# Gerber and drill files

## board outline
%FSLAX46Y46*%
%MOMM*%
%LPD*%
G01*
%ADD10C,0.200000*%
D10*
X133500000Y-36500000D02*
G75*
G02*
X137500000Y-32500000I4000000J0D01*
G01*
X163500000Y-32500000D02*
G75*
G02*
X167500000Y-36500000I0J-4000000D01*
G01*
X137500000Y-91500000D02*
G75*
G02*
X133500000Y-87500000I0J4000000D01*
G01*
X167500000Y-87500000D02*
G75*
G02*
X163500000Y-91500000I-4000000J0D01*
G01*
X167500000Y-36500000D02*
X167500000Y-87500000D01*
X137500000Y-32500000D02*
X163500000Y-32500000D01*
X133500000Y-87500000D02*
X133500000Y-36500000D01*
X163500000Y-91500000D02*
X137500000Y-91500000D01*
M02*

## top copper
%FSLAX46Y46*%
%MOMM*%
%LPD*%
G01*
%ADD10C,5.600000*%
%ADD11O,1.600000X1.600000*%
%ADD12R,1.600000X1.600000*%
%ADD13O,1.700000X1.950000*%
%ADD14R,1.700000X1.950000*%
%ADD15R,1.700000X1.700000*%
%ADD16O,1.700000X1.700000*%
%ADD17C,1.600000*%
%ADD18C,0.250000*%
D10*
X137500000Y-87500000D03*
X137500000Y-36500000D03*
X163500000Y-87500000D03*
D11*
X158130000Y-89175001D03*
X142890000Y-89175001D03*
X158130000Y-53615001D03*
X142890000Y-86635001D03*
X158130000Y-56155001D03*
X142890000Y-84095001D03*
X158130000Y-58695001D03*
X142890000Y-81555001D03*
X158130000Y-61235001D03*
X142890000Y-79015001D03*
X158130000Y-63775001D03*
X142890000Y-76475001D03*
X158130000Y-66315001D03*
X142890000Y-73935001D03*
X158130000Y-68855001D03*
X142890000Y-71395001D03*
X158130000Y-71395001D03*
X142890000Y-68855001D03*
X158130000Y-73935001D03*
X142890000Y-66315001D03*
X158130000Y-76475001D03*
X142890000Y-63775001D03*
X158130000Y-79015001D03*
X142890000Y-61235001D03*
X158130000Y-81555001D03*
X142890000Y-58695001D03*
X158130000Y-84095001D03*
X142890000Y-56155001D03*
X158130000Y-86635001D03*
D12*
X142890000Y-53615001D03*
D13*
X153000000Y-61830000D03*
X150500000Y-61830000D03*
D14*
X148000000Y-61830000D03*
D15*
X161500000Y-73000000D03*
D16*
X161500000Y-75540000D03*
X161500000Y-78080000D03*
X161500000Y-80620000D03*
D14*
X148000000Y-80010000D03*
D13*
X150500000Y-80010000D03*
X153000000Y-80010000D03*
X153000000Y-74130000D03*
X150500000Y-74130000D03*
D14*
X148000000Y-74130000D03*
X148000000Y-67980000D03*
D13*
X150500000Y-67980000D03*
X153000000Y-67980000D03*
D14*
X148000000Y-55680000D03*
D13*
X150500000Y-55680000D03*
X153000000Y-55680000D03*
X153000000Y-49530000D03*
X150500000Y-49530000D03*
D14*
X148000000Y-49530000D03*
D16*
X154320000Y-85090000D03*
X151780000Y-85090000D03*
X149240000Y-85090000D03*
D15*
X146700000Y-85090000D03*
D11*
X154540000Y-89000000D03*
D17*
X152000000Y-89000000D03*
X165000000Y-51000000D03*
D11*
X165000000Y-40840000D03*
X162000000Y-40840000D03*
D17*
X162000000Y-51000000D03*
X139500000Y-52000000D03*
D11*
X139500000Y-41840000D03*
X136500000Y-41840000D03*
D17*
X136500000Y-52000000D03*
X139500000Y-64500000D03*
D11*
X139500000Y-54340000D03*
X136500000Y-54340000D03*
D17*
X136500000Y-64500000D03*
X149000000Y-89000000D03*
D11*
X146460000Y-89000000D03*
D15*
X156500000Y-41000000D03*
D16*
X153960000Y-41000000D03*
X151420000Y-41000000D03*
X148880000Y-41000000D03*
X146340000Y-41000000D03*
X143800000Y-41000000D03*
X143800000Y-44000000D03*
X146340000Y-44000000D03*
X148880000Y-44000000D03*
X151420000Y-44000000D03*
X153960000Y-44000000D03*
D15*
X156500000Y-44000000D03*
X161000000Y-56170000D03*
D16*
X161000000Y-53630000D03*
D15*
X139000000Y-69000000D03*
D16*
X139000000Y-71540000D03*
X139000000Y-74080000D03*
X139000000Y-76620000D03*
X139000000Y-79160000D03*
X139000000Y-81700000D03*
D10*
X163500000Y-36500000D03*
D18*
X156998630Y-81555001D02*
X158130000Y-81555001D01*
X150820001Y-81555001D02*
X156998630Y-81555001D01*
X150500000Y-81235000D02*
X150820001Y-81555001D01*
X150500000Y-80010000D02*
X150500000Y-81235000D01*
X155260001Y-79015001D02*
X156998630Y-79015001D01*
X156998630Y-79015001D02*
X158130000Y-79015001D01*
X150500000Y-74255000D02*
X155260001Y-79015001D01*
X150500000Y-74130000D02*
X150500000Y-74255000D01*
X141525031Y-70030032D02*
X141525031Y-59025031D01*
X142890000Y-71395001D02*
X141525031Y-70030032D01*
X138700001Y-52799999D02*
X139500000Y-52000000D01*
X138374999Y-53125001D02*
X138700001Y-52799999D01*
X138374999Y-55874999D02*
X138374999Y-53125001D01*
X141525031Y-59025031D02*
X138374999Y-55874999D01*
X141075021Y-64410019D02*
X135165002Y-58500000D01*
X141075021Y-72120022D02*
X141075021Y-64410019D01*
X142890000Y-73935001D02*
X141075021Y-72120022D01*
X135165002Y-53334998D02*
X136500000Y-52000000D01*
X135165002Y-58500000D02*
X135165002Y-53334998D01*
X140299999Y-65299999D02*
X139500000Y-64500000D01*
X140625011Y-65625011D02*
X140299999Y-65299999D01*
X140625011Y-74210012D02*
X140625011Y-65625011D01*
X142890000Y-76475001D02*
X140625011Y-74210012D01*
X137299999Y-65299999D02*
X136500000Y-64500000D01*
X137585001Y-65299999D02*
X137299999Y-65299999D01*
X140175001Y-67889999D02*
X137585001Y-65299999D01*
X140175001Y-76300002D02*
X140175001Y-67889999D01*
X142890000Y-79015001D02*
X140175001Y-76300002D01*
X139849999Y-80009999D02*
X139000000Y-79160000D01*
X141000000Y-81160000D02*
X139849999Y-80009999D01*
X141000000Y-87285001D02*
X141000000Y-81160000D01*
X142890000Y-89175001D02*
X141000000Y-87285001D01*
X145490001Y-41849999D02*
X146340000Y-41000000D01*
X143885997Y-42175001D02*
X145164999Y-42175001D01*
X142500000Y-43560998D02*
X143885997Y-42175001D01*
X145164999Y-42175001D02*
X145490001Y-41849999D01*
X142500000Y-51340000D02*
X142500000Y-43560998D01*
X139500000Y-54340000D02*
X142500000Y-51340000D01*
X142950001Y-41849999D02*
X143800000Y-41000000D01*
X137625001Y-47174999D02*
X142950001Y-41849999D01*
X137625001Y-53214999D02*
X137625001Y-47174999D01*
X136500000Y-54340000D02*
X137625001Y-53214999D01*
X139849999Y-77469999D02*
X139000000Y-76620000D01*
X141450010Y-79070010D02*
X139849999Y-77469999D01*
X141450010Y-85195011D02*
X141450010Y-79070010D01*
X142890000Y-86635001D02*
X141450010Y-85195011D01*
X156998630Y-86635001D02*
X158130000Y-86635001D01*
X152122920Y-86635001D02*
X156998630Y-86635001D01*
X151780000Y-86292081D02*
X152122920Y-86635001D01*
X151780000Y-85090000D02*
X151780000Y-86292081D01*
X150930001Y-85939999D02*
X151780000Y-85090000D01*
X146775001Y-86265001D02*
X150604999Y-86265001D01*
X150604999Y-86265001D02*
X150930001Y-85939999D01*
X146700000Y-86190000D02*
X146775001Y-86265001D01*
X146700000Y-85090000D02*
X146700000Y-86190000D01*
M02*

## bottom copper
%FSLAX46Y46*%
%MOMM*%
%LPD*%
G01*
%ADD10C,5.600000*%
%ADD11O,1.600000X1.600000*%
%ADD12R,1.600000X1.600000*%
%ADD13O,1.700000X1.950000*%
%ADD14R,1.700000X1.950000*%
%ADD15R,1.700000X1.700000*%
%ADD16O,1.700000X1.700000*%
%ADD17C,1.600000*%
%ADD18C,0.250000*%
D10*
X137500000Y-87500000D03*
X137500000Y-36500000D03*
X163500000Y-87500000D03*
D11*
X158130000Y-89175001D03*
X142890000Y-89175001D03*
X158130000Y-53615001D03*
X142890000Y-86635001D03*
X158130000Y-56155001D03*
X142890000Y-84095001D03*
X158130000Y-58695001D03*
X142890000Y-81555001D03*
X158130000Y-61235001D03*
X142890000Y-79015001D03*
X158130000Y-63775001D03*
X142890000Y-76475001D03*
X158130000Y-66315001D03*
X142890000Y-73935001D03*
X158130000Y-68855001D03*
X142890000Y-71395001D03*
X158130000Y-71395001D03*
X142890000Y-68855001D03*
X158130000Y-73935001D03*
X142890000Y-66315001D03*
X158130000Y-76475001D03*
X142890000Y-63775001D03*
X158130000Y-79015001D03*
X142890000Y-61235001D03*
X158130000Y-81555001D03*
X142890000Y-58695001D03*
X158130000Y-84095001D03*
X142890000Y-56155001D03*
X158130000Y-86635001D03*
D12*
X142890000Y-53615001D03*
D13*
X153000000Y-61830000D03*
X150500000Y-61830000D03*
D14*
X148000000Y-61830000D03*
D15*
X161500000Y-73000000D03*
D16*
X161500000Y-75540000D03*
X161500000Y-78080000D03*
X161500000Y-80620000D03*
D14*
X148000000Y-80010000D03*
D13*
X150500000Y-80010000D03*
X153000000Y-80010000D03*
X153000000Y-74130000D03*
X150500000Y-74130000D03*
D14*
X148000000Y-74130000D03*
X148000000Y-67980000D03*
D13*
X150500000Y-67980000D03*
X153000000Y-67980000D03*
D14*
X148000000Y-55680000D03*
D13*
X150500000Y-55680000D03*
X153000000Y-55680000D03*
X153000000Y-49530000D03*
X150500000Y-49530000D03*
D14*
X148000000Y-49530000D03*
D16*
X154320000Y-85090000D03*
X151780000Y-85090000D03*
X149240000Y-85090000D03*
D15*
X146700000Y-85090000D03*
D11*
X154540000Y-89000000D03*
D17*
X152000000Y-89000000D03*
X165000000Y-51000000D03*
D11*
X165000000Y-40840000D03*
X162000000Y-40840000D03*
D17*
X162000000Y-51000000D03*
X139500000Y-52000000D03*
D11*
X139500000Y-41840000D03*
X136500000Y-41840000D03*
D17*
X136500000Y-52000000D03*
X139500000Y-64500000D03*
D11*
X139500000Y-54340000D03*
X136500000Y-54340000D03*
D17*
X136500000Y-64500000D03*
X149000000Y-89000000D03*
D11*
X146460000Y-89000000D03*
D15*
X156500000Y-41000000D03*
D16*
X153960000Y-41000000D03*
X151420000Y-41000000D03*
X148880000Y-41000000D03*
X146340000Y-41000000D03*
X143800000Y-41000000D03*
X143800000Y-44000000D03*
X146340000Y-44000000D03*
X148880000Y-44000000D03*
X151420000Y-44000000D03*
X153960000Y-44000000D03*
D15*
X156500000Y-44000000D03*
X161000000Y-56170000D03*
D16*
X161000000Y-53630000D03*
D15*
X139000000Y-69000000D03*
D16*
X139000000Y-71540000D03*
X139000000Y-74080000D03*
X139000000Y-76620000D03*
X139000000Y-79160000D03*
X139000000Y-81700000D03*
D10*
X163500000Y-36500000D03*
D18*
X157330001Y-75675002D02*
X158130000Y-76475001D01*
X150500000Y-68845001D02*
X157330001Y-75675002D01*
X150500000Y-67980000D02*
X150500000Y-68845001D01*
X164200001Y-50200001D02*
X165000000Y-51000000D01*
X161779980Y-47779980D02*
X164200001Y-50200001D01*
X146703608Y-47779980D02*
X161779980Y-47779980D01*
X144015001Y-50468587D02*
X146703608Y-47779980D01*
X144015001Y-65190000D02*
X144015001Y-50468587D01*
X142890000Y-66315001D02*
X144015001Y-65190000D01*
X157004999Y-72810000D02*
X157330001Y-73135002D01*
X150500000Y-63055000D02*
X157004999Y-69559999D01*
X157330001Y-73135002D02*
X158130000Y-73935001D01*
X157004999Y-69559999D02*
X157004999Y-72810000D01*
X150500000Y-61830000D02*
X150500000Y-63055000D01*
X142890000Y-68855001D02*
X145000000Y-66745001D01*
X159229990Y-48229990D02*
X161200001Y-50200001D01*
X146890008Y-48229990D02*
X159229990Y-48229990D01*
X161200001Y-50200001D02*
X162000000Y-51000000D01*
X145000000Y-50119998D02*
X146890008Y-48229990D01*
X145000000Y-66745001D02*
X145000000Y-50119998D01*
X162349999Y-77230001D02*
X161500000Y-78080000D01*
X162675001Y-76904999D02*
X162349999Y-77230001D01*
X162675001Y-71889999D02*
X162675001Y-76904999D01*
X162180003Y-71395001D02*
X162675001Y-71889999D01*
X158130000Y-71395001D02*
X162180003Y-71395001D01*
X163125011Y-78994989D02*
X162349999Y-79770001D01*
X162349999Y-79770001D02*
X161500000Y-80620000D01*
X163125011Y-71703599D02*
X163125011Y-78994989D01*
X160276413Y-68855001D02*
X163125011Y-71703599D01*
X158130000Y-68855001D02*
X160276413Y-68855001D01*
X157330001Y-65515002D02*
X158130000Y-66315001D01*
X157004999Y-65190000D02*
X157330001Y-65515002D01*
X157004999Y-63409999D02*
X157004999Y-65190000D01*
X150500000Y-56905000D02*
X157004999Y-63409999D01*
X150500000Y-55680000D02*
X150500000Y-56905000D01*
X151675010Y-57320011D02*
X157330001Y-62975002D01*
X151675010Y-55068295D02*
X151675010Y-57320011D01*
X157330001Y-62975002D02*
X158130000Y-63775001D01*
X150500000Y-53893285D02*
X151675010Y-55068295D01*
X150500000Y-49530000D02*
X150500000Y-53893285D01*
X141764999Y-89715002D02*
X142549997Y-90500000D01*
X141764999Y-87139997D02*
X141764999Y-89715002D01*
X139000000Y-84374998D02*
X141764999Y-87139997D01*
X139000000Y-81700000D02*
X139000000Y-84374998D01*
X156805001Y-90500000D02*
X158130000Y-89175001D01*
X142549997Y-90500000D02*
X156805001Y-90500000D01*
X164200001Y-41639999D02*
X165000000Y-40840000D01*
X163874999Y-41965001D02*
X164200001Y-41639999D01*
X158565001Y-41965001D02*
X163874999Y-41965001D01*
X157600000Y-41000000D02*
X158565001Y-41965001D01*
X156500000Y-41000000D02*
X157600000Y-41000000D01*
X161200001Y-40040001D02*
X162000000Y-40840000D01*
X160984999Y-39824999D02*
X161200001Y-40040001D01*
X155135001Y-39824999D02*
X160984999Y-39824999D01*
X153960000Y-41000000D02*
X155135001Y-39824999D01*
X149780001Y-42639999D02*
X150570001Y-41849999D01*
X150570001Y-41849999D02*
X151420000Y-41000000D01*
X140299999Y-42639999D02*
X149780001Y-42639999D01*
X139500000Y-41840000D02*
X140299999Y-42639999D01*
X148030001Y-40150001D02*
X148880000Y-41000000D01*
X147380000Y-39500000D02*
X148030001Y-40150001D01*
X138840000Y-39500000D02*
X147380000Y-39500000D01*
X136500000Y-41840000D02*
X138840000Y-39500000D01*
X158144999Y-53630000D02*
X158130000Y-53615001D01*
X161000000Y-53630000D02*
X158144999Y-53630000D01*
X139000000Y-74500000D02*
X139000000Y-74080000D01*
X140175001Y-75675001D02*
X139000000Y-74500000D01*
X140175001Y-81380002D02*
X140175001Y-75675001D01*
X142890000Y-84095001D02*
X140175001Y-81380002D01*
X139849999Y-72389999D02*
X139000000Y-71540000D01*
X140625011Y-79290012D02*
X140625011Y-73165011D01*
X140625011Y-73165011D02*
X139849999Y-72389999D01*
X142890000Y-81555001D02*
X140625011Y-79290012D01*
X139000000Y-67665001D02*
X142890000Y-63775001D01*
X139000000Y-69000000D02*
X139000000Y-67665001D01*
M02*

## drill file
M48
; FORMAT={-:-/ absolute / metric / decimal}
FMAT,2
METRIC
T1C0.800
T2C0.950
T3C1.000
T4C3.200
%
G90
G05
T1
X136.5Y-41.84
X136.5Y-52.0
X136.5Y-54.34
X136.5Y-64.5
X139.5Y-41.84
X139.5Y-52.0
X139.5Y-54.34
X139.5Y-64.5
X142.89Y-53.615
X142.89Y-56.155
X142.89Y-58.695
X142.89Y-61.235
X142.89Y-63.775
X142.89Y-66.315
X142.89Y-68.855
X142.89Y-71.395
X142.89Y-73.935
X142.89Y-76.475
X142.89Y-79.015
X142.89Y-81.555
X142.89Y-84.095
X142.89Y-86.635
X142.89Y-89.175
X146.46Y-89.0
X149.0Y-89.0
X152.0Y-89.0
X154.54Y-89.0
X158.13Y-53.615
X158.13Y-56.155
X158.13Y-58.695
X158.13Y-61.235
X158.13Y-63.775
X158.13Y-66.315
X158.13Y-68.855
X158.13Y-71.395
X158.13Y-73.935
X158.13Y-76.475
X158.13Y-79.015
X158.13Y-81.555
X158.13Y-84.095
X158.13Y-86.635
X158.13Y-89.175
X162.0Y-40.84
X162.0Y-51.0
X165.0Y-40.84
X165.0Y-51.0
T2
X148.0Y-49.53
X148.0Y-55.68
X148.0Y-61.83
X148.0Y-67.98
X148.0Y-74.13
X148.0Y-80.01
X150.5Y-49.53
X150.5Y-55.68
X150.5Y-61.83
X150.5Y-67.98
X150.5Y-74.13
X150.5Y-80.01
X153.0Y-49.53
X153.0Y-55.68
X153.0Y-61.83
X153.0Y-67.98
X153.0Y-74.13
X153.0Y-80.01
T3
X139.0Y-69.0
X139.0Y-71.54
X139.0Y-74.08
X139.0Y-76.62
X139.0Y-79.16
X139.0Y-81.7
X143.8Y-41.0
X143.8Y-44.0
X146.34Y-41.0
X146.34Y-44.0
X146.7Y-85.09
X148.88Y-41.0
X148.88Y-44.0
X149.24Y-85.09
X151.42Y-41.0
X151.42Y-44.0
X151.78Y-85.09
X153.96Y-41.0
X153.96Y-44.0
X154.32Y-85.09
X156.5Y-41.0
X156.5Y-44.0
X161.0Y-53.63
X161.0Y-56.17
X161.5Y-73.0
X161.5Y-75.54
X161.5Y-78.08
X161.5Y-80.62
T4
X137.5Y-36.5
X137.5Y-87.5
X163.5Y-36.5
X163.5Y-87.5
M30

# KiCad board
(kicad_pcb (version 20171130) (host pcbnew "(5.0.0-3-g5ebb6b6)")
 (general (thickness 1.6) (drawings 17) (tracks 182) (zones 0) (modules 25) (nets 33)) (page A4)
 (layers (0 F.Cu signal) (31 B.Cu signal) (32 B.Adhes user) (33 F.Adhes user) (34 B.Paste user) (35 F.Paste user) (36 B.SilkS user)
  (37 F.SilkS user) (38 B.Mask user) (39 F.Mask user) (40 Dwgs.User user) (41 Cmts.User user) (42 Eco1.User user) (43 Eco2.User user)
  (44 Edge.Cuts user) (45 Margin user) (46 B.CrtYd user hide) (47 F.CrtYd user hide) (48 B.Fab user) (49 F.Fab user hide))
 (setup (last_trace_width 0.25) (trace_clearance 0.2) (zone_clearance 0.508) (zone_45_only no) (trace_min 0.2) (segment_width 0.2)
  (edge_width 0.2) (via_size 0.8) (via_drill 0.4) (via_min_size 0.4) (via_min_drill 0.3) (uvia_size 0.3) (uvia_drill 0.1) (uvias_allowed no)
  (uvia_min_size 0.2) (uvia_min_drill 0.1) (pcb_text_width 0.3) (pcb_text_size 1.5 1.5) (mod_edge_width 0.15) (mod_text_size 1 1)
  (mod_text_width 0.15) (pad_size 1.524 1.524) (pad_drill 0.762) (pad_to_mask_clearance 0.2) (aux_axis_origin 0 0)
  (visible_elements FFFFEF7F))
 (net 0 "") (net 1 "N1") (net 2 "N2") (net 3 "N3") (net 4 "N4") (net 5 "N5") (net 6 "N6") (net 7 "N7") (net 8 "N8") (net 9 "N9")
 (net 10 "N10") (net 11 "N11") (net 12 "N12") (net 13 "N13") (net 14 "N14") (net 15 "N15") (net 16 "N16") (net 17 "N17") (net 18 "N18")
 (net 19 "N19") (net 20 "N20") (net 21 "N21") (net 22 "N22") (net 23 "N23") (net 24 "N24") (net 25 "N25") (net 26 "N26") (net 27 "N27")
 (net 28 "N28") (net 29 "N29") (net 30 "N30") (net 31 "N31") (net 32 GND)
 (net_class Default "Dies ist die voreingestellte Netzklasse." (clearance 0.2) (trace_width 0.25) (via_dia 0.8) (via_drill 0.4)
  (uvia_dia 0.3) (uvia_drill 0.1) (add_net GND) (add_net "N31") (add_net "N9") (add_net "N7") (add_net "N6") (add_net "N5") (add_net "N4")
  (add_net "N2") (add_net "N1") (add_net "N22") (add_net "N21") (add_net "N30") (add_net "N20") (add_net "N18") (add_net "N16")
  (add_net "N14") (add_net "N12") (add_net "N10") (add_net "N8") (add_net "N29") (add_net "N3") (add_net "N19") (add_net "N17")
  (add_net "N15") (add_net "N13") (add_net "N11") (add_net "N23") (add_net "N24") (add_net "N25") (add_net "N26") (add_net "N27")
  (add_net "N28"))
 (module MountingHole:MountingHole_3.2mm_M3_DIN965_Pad (layer F.Cu) (at 137.5 87.5)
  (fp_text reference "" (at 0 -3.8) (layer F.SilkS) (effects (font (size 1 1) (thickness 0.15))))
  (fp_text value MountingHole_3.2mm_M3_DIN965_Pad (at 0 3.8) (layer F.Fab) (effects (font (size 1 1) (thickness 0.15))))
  (pad 1 thru_hole circle (at 0 0) (size 5.6 5.6) (drill 3.2) (layers *.Cu *.Mask)))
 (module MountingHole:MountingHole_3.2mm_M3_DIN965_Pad (layer F.Cu) (at 137.5 36.5)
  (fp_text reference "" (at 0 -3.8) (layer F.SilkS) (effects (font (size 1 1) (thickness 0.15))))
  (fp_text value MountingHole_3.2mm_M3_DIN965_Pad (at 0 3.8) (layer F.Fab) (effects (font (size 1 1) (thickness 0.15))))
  (pad 1 thru_hole circle (at 0 0) (size 5.6 5.6) (drill 3.2) (layers *.Cu *.Mask)))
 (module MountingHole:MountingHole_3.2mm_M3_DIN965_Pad (layer F.Cu) (at 163.5 87.5)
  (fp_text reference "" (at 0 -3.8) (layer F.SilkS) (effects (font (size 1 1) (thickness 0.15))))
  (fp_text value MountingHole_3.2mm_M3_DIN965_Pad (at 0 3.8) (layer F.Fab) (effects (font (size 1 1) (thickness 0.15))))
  (pad 1 thru_hole circle (at 0 0) (size 5.6 5.6) (drill 3.2) (layers *.Cu *.Mask)))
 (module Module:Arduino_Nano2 (layer F.Cu) (at 142.89 53.615001)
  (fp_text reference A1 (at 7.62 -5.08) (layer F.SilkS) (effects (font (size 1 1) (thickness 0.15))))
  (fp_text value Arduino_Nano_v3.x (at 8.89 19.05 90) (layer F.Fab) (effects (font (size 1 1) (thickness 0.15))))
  (pad 16 thru_hole oval (at 15.24 35.56) (size 1.6 1.6) (drill 0.8) (layers *.Cu *.Mask) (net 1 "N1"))
  (pad 15 thru_hole oval (at 0 35.56) (size 1.6 1.6) (drill 0.8) (layers *.Cu *.Mask) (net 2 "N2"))
  (pad 30 thru_hole oval (at 15.24 0) (size 1.6 1.6) (drill 0.8) (layers *.Cu *.Mask) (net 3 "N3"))
  (pad 14 thru_hole oval (at 0 33.02) (size 1.6 1.6) (drill 0.8) (layers *.Cu *.Mask) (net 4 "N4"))
  (pad 29 thru_hole oval (at 15.24 2.54) (size 1.6 1.6) (drill 0.8) (layers *.Cu *.Mask))
  (pad 13 thru_hole oval (at 0 30.48) (size 1.6 1.6) (drill 0.8) (layers *.Cu *.Mask) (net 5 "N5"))
  (pad 28 thru_hole oval (at 15.24 5.08) (size 1.6 1.6) (drill 0.8) (layers *.Cu *.Mask))
  (pad 12 thru_hole oval (at 0 27.94) (size 1.6 1.6) (drill 0.8) (layers *.Cu *.Mask) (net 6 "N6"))
  (pad 27 thru_hole oval (at 15.24 7.62) (size 1.6 1.6) (drill 0.8) (layers *.Cu *.Mask))
  (pad 11 thru_hole oval (at 0 25.4) (size 1.6 1.6) (drill 0.8) (layers *.Cu *.Mask) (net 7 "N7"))
  (pad 26 thru_hole oval (at 15.24 10.16) (size 1.6 1.6) (drill 0.8) (layers *.Cu *.Mask) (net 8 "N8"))
  (pad 10 thru_hole oval (at 0 22.86) (size 1.6 1.6) (drill 0.8) (layers *.Cu *.Mask) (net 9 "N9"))
  (pad 25 thru_hole oval (at 15.24 12.7) (size 1.6 1.6) (drill 0.8) (layers *.Cu *.Mask) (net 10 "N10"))
  (pad 9 thru_hole oval (at 0 20.32) (size 1.6 1.6) (drill 0.8) (layers *.Cu *.Mask) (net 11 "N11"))
  (pad 24 thru_hole oval (at 15.24 15.24) (size 1.6 1.6) (drill 0.8) (layers *.Cu *.Mask) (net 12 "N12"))
  (pad 8 thru_hole oval (at 0 17.78) (size 1.6 1.6) (drill 0.8) (layers *.Cu *.Mask) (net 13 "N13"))
  (pad 23 thru_hole oval (at 15.24 17.78) (size 1.6 1.6) (drill 0.8) (layers *.Cu *.Mask) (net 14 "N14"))
  (pad 7 thru_hole oval (at 0 15.24) (size 1.6 1.6) (drill 0.8) (layers *.Cu *.Mask) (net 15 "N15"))
  (pad 22 thru_hole oval (at 15.24 20.32) (size 1.6 1.6) (drill 0.8) (layers *.Cu *.Mask) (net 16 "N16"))
  (pad 6 thru_hole oval (at 0 12.7) (size 1.6 1.6) (drill 0.8) (layers *.Cu *.Mask) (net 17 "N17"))
  (pad 21 thru_hole oval (at 15.24 22.86) (size 1.6 1.6) (drill 0.8) (layers *.Cu *.Mask) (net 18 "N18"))
  (pad 5 thru_hole oval (at 0 10.16) (size 1.6 1.6) (drill 0.8) (layers *.Cu *.Mask) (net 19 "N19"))
  (pad 20 thru_hole oval (at 15.24 25.4) (size 1.6 1.6) (drill 0.8) (layers *.Cu *.Mask) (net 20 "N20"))
  (pad 4 thru_hole oval (at 0 7.62) (size 1.6 1.6) (drill 0.8) (layers *.Cu *.Mask))
  (pad 19 thru_hole oval (at 15.24 27.94) (size 1.6 1.6) (drill 0.8) (layers *.Cu *.Mask) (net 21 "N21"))
  (pad 3 thru_hole oval (at 0 5.08) (size 1.6 1.6) (drill 0.8) (layers *.Cu *.Mask))
  (pad 18 thru_hole oval (at 15.24 30.48) (size 1.6 1.6) (drill 0.8) (layers *.Cu *.Mask))
  (pad 2 thru_hole oval (at 0 2.54) (size 1.6 1.6) (drill 0.8) (layers *.Cu *.Mask))
  (pad 17 thru_hole oval (at 15.24 33.02) (size 1.6 1.6) (drill 0.8) (layers *.Cu *.Mask) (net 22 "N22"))
  (pad 1 thru_hole rect (at 0 0) (size 1.6 1.6) (drill 0.8) (layers *.Cu *.Mask)))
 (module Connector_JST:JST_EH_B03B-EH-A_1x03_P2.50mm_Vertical (layer F.Cu) (at 148 61.83)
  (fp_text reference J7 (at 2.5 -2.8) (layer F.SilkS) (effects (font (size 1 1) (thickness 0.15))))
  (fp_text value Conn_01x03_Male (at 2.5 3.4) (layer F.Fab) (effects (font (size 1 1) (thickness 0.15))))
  (pad 3 thru_hole oval (at 5 0) (size 1.7 1.95) (drill 0.95) (layers *.Cu *.Mask))
  (pad 2 thru_hole oval (at 2.5 0) (size 1.7 1.95) (drill 0.95) (layers *.Cu *.Mask) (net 16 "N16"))
  (pad 1 thru_hole rect (at 0 0) (size 1.7 1.95) (drill 0.95) (layers *.Cu *.Mask)))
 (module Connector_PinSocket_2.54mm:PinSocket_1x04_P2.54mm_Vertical (layer F.Cu) (at 161.5 73)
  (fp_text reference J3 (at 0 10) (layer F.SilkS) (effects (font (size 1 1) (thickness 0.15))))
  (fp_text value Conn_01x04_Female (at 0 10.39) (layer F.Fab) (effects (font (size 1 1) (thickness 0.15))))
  (pad 1 thru_hole rect (at 0 0) (size 1.7 1.7) (drill 1) (layers *.Cu *.Mask))
  (pad 2 thru_hole oval (at 0 2.54) (size 1.7 1.7) (drill 1) (layers *.Cu *.Mask))
  (pad 3 thru_hole oval (at 0 5.08) (size 1.7 1.7) (drill 1) (layers *.Cu *.Mask) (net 14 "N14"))
  (pad 4 thru_hole oval (at 0 7.62) (size 1.7 1.7) (drill 1) (layers *.Cu *.Mask) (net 12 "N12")))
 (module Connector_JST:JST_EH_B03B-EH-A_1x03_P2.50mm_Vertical (layer F.Cu) (at 148 80.01)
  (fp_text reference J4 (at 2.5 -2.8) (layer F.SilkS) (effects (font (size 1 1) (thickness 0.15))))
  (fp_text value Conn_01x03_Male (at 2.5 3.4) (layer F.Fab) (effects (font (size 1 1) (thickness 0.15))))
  (pad 1 thru_hole rect (at 0 0) (size 1.7 1.95) (drill 0.95) (layers *.Cu *.Mask))
  (pad 2 thru_hole oval (at 2.5 0) (size 1.7 1.95) (drill 0.95) (layers *.Cu *.Mask) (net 21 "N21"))
  (pad 3 thru_hole oval (at 5 0) (size 1.7 1.95) (drill 0.95) (layers *.Cu *.Mask)))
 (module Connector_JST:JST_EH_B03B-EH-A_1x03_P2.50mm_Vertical (layer F.Cu) (at 148 74.13)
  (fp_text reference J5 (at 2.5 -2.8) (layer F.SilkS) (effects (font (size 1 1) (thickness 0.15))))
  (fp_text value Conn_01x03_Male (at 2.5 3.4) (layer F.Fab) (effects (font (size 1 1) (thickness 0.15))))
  (pad 3 thru_hole oval (at 5 0) (size 1.7 1.95) (drill 0.95) (layers *.Cu *.Mask))
  (pad 2 thru_hole oval (at 2.5 0) (size 1.7 1.95) (drill 0.95) (layers *.Cu *.Mask) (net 20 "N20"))
  (pad 1 thru_hole rect (at 0 0) (size 1.7 1.95) (drill 0.95) (layers *.Cu *.Mask)))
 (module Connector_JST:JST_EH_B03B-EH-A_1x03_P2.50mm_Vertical (layer F.Cu) (at 148 67.98)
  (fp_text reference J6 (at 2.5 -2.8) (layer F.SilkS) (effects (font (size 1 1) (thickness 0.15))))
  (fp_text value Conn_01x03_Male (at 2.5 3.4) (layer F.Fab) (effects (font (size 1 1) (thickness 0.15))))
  (pad 1 thru_hole rect (at 0 0) (size 1.7 1.95) (drill 0.95) (layers *.Cu *.Mask))
  (pad 2 thru_hole oval (at 2.5 0) (size 1.7 1.95) (drill 0.95) (layers *.Cu *.Mask) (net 18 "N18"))
  (pad 3 thru_hole oval (at 5 0) (size 1.7 1.95) (drill 0.95) (layers *.Cu *.Mask)))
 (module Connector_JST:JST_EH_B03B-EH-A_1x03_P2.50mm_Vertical (layer F.Cu) (at 148 55.68)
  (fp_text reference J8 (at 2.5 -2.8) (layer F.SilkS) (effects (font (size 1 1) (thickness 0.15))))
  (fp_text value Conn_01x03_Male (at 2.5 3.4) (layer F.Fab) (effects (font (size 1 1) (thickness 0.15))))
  (pad 1 thru_hole rect (at 0 0) (size 1.7 1.95) (drill 0.95) (layers *.Cu *.Mask))
  (pad 2 thru_hole oval (at 2.5 0) (size 1.7 1.95) (drill 0.95) (layers *.Cu *.Mask) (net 10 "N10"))
  (pad 3 thru_hole oval (at 5 0) (size 1.7 1.95) (drill 0.95) (layers *.Cu *.Mask)))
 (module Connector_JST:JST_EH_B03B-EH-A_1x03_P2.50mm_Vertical (layer F.Cu) (at 148 49.53)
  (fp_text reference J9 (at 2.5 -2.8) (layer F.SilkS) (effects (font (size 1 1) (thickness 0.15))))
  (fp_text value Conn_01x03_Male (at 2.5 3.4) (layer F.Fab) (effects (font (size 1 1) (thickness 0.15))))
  (pad 3 thru_hole oval (at 5 0) (size 1.7 1.95) (drill 0.95) (layers *.Cu *.Mask))
  (pad 2 thru_hole oval (at 2.5 0) (size 1.7 1.95) (drill 0.95) (layers *.Cu *.Mask) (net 8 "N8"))
  (pad 1 thru_hole rect (at 0 0) (size 1.7 1.95) (drill 0.95) (layers *.Cu *.Mask)))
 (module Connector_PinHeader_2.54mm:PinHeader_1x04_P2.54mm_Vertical (layer F.Cu) (at 146.7 85.09 90)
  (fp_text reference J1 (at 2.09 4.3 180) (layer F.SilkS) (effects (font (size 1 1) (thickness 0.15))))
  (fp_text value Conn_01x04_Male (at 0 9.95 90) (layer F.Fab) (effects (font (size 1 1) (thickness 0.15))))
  (pad 4 thru_hole oval (at 0 7.62 90) (size 1.7 1.7) (drill 1) (layers *.Cu *.Mask))
  (pad 3 thru_hole oval (at 0 5.08 90) (size 1.7 1.7) (drill 1) (layers *.Cu *.Mask) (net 22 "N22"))
  (pad 2 thru_hole oval (at 0 2.54 90) (size 1.7 1.7) (drill 1) (layers *.Cu *.Mask))
  (pad 1 thru_hole rect (at 0 0 90) (size 1.7 1.7) (drill 1) (layers *.Cu *.Mask) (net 22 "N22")))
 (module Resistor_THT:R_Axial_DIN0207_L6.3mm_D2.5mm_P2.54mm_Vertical (layer F.Cu) (at 152 89)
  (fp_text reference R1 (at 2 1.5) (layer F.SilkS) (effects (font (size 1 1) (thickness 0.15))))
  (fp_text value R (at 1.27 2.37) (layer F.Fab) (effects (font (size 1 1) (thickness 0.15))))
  (pad 2 thru_hole oval (at 2.54 0) (size 1.6 1.6) (drill 0.8) (layers *.Cu *.Mask))
  (pad 1 thru_hole circle (at 0 0) (size 1.6 1.6) (drill 0.8) (layers *.Cu *.Mask)))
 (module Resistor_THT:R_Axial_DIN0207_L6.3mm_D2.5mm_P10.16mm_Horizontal (layer F.Cu) (at 165 51 90)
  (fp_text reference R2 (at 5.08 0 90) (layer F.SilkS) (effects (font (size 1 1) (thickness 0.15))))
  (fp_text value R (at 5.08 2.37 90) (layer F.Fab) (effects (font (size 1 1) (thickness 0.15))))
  (pad 1 thru_hole circle (at 0 0 90) (size 1.6 1.6) (drill 0.8) (layers *.Cu *.Mask) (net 17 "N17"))
  (pad 2 thru_hole oval (at 10.16 0 90) (size 1.6 1.6) (drill 0.8) (layers *.Cu *.Mask) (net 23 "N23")))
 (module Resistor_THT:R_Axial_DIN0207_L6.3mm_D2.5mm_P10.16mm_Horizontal (layer F.Cu) (at 162 51 90)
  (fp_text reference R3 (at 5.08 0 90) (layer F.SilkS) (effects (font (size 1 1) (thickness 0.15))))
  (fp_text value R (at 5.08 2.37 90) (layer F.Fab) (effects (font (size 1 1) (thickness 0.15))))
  (pad 2 thru_hole oval (at 10.16 0 90) (size 1.6 1.6) (drill 0.8) (layers *.Cu *.Mask) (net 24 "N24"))
  (pad 1 thru_hole circle (at 0 0 90) (size 1.6 1.6) (drill 0.8) (layers *.Cu *.Mask) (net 15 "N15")))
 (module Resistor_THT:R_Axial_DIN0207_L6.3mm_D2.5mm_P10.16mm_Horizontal (layer F.Cu) (at 139.5 52 90)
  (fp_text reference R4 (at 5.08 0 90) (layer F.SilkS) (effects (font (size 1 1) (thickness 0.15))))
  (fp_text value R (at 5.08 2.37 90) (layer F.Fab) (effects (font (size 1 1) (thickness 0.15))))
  (pad 1 thru_hole circle (at 0 0 90) (size 1.6 1.6) (drill 0.8) (layers *.Cu *.Mask) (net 13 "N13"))
  (pad 2 thru_hole oval (at 10.16 0 90) (size 1.6 1.6) (drill 0.8) (layers *.Cu *.Mask) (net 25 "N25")))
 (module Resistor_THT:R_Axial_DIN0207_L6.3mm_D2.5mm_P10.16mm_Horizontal (layer F.Cu) (at 136.5 52 90)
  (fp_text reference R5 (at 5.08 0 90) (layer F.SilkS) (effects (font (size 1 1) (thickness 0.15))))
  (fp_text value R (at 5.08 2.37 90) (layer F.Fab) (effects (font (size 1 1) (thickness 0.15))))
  (pad 2 thru_hole oval (at 10.16 0 90) (size 1.6 1.6) (drill 0.8) (layers *.Cu *.Mask) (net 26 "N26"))
  (pad 1 thru_hole circle (at 0 0 90) (size 1.6 1.6) (drill 0.8) (layers *.Cu *.Mask) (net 11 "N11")))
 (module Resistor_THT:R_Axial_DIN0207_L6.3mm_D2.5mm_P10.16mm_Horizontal (layer F.Cu) (at 139.5 64.5 90)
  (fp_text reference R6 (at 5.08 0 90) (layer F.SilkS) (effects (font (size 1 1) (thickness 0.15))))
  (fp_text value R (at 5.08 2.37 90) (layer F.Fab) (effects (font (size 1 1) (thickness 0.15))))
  (pad 1 thru_hole circle (at 0 0 90) (size 1.6 1.6) (drill 0.8) (layers *.Cu *.Mask) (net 9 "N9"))
  (pad 2 thru_hole oval (at 10.16 0 90) (size 1.6 1.6) (drill 0.8) (layers *.Cu *.Mask) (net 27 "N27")))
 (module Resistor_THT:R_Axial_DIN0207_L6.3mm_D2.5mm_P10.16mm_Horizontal (layer F.Cu) (at 136.5 64.5 90)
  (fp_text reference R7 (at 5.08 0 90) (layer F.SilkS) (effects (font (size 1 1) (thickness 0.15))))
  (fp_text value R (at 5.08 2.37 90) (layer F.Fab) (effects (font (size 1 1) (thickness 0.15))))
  (pad 2 thru_hole oval (at 10.16 0 90) (size 1.6 1.6) (drill 0.8) (layers *.Cu *.Mask) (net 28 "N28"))
  (pad 1 thru_hole circle (at 0 0 90) (size 1.6 1.6) (drill 0.8) (layers *.Cu *.Mask) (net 7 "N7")))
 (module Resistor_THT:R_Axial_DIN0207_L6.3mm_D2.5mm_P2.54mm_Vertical (layer F.Cu) (at 149 89 180)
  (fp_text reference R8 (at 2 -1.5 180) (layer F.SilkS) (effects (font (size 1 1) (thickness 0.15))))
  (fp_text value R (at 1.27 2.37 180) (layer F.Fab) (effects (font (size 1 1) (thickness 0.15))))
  (pad 1 thru_hole circle (at 0 0 180) (size 1.6 1.6) (drill 0.8) (layers *.Cu *.Mask))
  (pad 2 thru_hole oval (at 2.54 0 180) (size 1.6 1.6) (drill 0.8) (layers *.Cu *.Mask)))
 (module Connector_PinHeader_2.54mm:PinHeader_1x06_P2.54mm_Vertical (layer F.Cu) (at 156.5 41 270)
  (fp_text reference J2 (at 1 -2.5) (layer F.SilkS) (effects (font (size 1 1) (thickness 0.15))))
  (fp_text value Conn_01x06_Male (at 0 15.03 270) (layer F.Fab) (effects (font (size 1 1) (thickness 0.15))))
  (pad 1 thru_hole rect (at 0 0 270) (size 1.7 1.7) (drill 1) (layers *.Cu *.Mask) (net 23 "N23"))
  (pad 2 thru_hole oval (at 0 2.54 270) (size 1.7 1.7) (drill 1) (layers *.Cu *.Mask) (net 24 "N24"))
  (pad 3 thru_hole oval (at 0 5.08 270) (size 1.7 1.7) (drill 1) (layers *.Cu *.Mask) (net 25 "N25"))
  (pad 4 thru_hole oval (at 0 7.62 270) (size 1.7 1.7) (drill 1) (layers *.Cu *.Mask) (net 26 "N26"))
  (pad 5 thru_hole oval (at 0 10.16 270) (size 1.7 1.7) (drill 1) (layers *.Cu *.Mask) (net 27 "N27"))
  (pad 6 thru_hole oval (at 0 12.7 270) (size 1.7 1.7) (drill 1) (layers *.Cu *.Mask) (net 28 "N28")))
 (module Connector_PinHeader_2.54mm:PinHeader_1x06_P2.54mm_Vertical (layer F.Cu) (at 156.5 44 270)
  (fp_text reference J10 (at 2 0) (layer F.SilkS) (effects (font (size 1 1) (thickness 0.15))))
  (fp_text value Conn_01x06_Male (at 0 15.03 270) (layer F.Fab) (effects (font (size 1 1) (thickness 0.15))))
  (pad 6 thru_hole oval (at 0 12.7 270) (size 1.7 1.7) (drill 1) (layers *.Cu *.Mask))
  (pad 5 thru_hole oval (at 0 10.16 270) (size 1.7 1.7) (drill 1) (layers *.Cu *.Mask))
  (pad 4 thru_hole oval (at 0 7.62 270) (size 1.7 1.7) (drill 1) (layers *.Cu *.Mask))
  (pad 3 thru_hole oval (at 0 5.08 270) (size 1.7 1.7) (drill 1) (layers *.Cu *.Mask))
  (pad 2 thru_hole oval (at 0 2.54 270) (size 1.7 1.7) (drill 1) (layers *.Cu *.Mask))
  (pad 1 thru_hole rect (at 0 0 270) (size 1.7 1.7) (drill 1) (layers *.Cu *.Mask)))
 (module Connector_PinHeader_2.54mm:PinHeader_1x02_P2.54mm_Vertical (layer F.Cu) (at 161 56.17 180)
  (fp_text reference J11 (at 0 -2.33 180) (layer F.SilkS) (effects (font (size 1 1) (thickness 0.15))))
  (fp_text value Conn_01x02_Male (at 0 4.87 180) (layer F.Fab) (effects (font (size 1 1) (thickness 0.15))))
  (pad 1 thru_hole rect (at 0 0 180) (size 1.7 1.7) (drill 1) (layers *.Cu *.Mask))
  (pad 2 thru_hole oval (at 0 2.54 180) (size 1.7 1.7) (drill 1) (layers *.Cu *.Mask) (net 3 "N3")))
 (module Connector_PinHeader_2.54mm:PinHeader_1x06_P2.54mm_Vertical (layer F.Cu) (at 139 69)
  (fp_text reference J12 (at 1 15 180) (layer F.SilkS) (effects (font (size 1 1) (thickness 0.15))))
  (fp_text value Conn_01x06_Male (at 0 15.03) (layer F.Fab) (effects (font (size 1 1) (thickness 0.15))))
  (pad 1 thru_hole rect (at 0 0) (size 1.7 1.7) (drill 1) (layers *.Cu *.Mask) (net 19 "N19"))
  (pad 2 thru_hole oval (at 0 2.54) (size 1.7 1.7) (drill 1) (layers *.Cu *.Mask) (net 6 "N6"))
  (pad 3 thru_hole oval (at 0 5.08) (size 1.7 1.7) (drill 1) (layers *.Cu *.Mask) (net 5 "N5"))
  (pad 4 thru_hole oval (at 0 7.62) (size 1.7 1.7) (drill 1) (layers *.Cu *.Mask) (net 4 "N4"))
  (pad 5 thru_hole oval (at 0 10.16) (size 1.7 1.7) (drill 1) (layers *.Cu *.Mask) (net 2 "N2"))
  (pad 6 thru_hole oval (at 0 12.7) (size 1.7 1.7) (drill 1) (layers *.Cu *.Mask) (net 1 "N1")))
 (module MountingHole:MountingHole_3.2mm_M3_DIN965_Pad (layer F.Cu) (at 163.5 36.5)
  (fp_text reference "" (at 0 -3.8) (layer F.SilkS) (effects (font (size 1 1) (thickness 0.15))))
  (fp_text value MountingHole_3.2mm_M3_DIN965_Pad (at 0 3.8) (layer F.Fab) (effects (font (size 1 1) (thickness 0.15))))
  (pad 1 thru_hole circle (at 0 0) (size 5.6 5.6) (drill 3.2) (layers *.Cu *.Mask)))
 (gr_arc (start 137.5 36.5) (end 137.5 32.5) (angle -90) (layer Edge.Cuts) (width 0.2))
 (gr_arc (start 163.5 36.5) (end 167.5 36.5) (angle -90) (layer Edge.Cuts) (width 0.2))
 (gr_arc (start 137.5 87.5) (end 133.5 87.5) (angle -90) (layer Edge.Cuts) (width 0.2))
 (gr_arc (start 163.5 87.5) (end 163.5 91.5) (angle -90) (layer Edge.Cuts) (width 0.2))
 (gr_line (start 167.5 36.5) (end 167.5 87.5) (layer Edge.Cuts) (width 0.2))
 (gr_line (start 137.5 32.5) (end 163.5 32.5) (layer Edge.Cuts) (width 0.2))
 (gr_line (start 133.5 87.5) (end 133.5 36.5) (layer Edge.Cuts) (width 0.2))
 (gr_line (start 163.5 91.5) (end 137.5 91.5) (layer Edge.Cuts) (width 0.2))
 (segment (start 156.99863 81.555001) (end 158.13 81.555001) (width 0.25) (layer F.Cu) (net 21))
 (segment (start 150.820001 81.555001) (end 156.99863 81.555001) (width 0.25) (layer F.Cu) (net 21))
 (segment (start 150.5 81.235) (end 150.820001 81.555001) (width 0.25) (layer F.Cu) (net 21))
 (segment (start 150.5 80.01) (end 150.5 81.235) (width 0.25) (layer F.Cu) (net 21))
 (segment (start 155.260001 79.015001) (end 156.99863 79.015001) (width 0.25) (layer F.Cu) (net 20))
 (segment (start 156.99863 79.015001) (end 158.13 79.015001) (width 0.25) (layer F.Cu) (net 20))
 (segment (start 150.5 74.255) (end 155.260001 79.015001) (width 0.25) (layer F.Cu) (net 20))
 (segment (start 150.5 74.13) (end 150.5 74.255) (width 0.25) (layer F.Cu) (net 20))
 (segment (start 157.330001 75.675002) (end 158.13 76.475001) (width 0.25) (layer B.Cu) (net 18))
 (segment (start 150.5 68.845001) (end 157.330001 75.675002) (width 0.25) (layer B.Cu) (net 18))
 (segment (start 150.5 67.98) (end 150.5 68.845001) (width 0.25) (layer B.Cu) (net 18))
 (segment (start 164.200001 50.200001) (end 165 51) (width 0.25) (layer B.Cu) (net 17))
 (segment (start 161.77998 47.77998) (end 164.200001 50.200001) (width 0.25) (layer B.Cu) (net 17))
 (segment (start 146.703608 47.77998) (end 161.77998 47.77998) (width 0.25) (layer B.Cu) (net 17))
 (segment (start 144.015001 50.468587) (end 146.703608 47.77998) (width 0.25) (layer B.Cu) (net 17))
 (segment (start 144.015001 65.19) (end 144.015001 50.468587) (width 0.25) (layer B.Cu) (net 17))
 (segment (start 142.89 66.315001) (end 144.015001 65.19) (width 0.25) (layer B.Cu) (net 17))
 (segment (start 157.004999 72.81) (end 157.330001 73.135002) (width 0.25) (layer B.Cu) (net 16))
 (segment (start 150.5 63.055) (end 157.004999 69.559999) (width 0.25) (layer B.Cu) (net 16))
 (segment (start 157.330001 73.135002) (end 158.13 73.935001) (width 0.25) (layer B.Cu) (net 16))
 (segment (start 157.004999 69.559999) (end 157.004999 72.81) (width 0.25) (layer B.Cu) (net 16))
 (segment (start 150.5 61.83) (end 150.5 63.055) (width 0.25) (layer B.Cu) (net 16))
 (segment (start 142.89 68.855001) (end 145 66.745001) (width 0.25) (layer B.Cu) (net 15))
 (segment (start 159.22999 48.22999) (end 161.200001 50.200001) (width 0.25) (layer B.Cu) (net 15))
 (segment (start 146.890008 48.22999) (end 159.22999 48.22999) (width 0.25) (layer B.Cu) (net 15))
 (segment (start 161.200001 50.200001) (end 162 51) (width 0.25) (layer B.Cu) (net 15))
 (segment (start 145 50.119998) (end 146.890008 48.22999) (width 0.25) (layer B.Cu) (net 15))
 (segment (start 145 66.745001) (end 145 50.119998) (width 0.25) (layer B.Cu) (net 15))
 (segment (start 162.349999 77.230001) (end 161.5 78.08) (width 0.25) (layer B.Cu) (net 14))
 (segment (start 162.675001 76.904999) (end 162.349999 77.230001) (width 0.25) (layer B.Cu) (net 14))
 (segment (start 162.675001 71.889999) (end 162.675001 76.904999) (width 0.25) (layer B.Cu) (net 14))
 (segment (start 162.180003 71.395001) (end 162.675001 71.889999) (width 0.25) (layer B.Cu) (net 14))
 (segment (start 158.13 71.395001) (end 162.180003 71.395001) (width 0.25) (layer B.Cu) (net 14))
 (segment (start 141.525031 70.030032) (end 141.525031 59.025031) (width 0.25) (layer F.Cu) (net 13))
 (segment (start 142.89 71.395001) (end 141.525031 70.030032) (width 0.25) (layer F.Cu) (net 13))
 (segment (start 138.700001 52.799999) (end 139.5 52) (width 0.25) (layer F.Cu) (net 13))
 (segment (start 138.374999 53.125001) (end 138.700001 52.799999) (width 0.25) (layer F.Cu) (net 13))
 (segment (start 138.374999 55.874999) (end 138.374999 53.125001) (width 0.25) (layer F.Cu) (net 13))
 (segment (start 141.525031 59.025031) (end 138.374999 55.874999) (width 0.25) (layer F.Cu) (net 13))
 (segment (start 163.125011 78.994989) (end 162.349999 79.770001) (width 0.25) (layer B.Cu) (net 12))
 (segment (start 162.349999 79.770001) (end 161.5 80.62) (width 0.25) (layer B.Cu) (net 12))
 (segment (start 163.125011 71.703599) (end 163.125011 78.994989) (width 0.25) (layer B.Cu) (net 12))
 (segment (start 160.276413 68.855001) (end 163.125011 71.703599) (width 0.25) (layer B.Cu) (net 12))
 (segment (start 158.13 68.855001) (end 160.276413 68.855001) (width 0.25) (layer B.Cu) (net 12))
 (segment (start 141.075021 64.410019) (end 135.165002 58.5) (width 0.25) (layer F.Cu) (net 11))
 (segment (start 141.075021 72.120022) (end 141.075021 64.410019) (width 0.25) (layer F.Cu) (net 11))
 (segment (start 142.89 73.935001) (end 141.075021 72.120022) (width 0.25) (layer F.Cu) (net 11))
 (segment (start 135.165002 53.334998) (end 136.5 52) (width 0.25) (layer F.Cu) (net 11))
 (segment (start 135.165002 58.5) (end 135.165002 53.334998) (width 0.25) (layer F.Cu) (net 11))
 (segment (start 157.330001 65.515002) (end 158.13 66.315001) (width 0.25) (layer B.Cu) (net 10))
 (segment (start 157.004999 65.19) (end 157.330001 65.515002) (width 0.25) (layer B.Cu) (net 10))
 (segment (start 157.004999 63.409999) (end 157.004999 65.19) (width 0.25) (layer B.Cu) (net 10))
 (segment (start 150.5 56.905) (end 157.004999 63.409999) (width 0.25) (layer B.Cu) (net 10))
 (segment (start 150.5 55.68) (end 150.5 56.905) (width 0.25) (layer B.Cu) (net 10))
 (segment (start 140.299999 65.299999) (end 139.5 64.5) (width 0.25) (layer F.Cu) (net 9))
 (segment (start 140.625011 65.625011) (end 140.299999 65.299999) (width 0.25) (layer F.Cu) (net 9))
 (segment (start 140.625011 74.210012) (end 140.625011 65.625011) (width 0.25) (layer F.Cu) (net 9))
 (segment (start 142.89 76.475001) (end 140.625011 74.210012) (width 0.25) (layer F.Cu) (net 9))
 (segment (start 151.67501 57.320011) (end 157.330001 62.975002) (width 0.25) (layer B.Cu) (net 8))
 (segment (start 151.67501 55.068295) (end 151.67501 57.320011) (width 0.25) (layer B.Cu) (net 8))
 (segment (start 157.330001 62.975002) (end 158.13 63.775001) (width 0.25) (layer B.Cu) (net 8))
 (segment (start 150.5 53.893285) (end 151.67501 55.068295) (width 0.25) (layer B.Cu) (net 8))
 (segment (start 150.5 49.53) (end 150.5 53.893285) (width 0.25) (layer B.Cu) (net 8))
 (segment (start 137.299999 65.299999) (end 136.5 64.5) (width 0.25) (layer F.Cu) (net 7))
 (segment (start 137.585001 65.299999) (end 137.299999 65.299999) (width 0.25) (layer F.Cu) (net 7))
 (segment (start 140.175001 67.889999) (end 137.585001 65.299999) (width 0.25) (layer F.Cu) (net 7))
 (segment (start 140.175001 76.300002) (end 140.175001 67.889999) (width 0.25) (layer F.Cu) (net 7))
 (segment (start 142.89 79.015001) (end 140.175001 76.300002) (width 0.25) (layer F.Cu) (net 7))
 (segment (start 139.849999 80.009999) (end 139 79.16) (width 0.25) (layer F.Cu) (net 2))
 (segment (start 141 81.16) (end 139.849999 80.009999) (width 0.25) (layer F.Cu) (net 2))
 (segment (start 141 87.285001) (end 141 81.16) (width 0.25) (layer F.Cu) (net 2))
 (segment (start 142.89 89.175001) (end 141 87.285001) (width 0.25) (layer F.Cu) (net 2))
 (segment (start 141.764999 89.715002) (end 142.549997 90.5) (width 0.25) (layer B.Cu) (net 1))
 (segment (start 141.764999 87.139997) (end 141.764999 89.715002) (width 0.25) (layer B.Cu) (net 1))
 (segment (start 139 84.374998) (end 141.764999 87.139997) (width 0.25) (layer B.Cu) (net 1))
 (segment (start 139 81.7) (end 139 84.374998) (width 0.25) (layer B.Cu) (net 1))
 (segment (start 156.805001 90.5) (end 158.13 89.175001) (width 0.25) (layer B.Cu) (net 1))
 (segment (start 142.549997 90.5) (end 156.805001 90.5) (width 0.25) (layer B.Cu) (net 1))
 (segment (start 164.200001 41.639999) (end 165 40.84) (width 0.25) (layer B.Cu) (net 23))
 (segment (start 163.874999 41.965001) (end 164.200001 41.639999) (width 0.25) (layer B.Cu) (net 23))
 (segment (start 158.565001 41.965001) (end 163.874999 41.965001) (width 0.25) (layer B.Cu) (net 23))
 (segment (start 157.6 41) (end 158.565001 41.965001) (width 0.25) (layer B.Cu) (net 23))
 (segment (start 156.5 41) (end 157.6 41) (width 0.25) (layer B.Cu) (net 23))
 (segment (start 161.200001 40.040001) (end 162 40.84) (width 0.25) (layer B.Cu) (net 24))
 (segment (start 160.984999 39.824999) (end 161.200001 40.040001) (width 0.25) (layer B.Cu) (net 24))
 (segment (start 155.135001 39.824999) (end 160.984999 39.824999) (width 0.25) (layer B.Cu) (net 24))
 (segment (start 153.96 41) (end 155.135001 39.824999) (width 0.25) (layer B.Cu) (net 24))
 (segment (start 149.780001 42.639999) (end 150.570001 41.849999) (width 0.25) (layer B.Cu) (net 25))
 (segment (start 150.570001 41.849999) (end 151.42 41) (width 0.25) (layer B.Cu) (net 25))
 (segment (start 140.299999 42.639999) (end 149.780001 42.639999) (width 0.25) (layer B.Cu) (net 25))
 (segment (start 139.5 41.84) (end 140.299999 42.639999) (width 0.25) (layer B.Cu) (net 25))
 (segment (start 148.030001 40.150001) (end 148.88 41) (width 0.25) (layer B.Cu) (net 26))
 (segment (start 147.38 39.5) (end 148.030001 40.150001) (width 0.25) (layer B.Cu) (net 26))
 (segment (start 138.84 39.5) (end 147.38 39.5) (width 0.25) (layer B.Cu) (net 26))
 (segment (start 136.5 41.84) (end 138.84 39.5) (width 0.25) (layer B.Cu) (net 26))
 (segment (start 145.490001 41.849999) (end 146.34 41) (width 0.25) (layer F.Cu) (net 27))
 (segment (start 143.885997 42.175001) (end 145.164999 42.175001) (width 0.25) (layer F.Cu) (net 27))
 (segment (start 142.5 43.560998) (end 143.885997 42.175001) (width 0.25) (layer F.Cu) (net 27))
 (segment (start 145.164999 42.175001) (end 145.490001 41.849999) (width 0.25) (layer F.Cu) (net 27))
 (segment (start 142.5 51.34) (end 142.5 43.560998) (width 0.25) (layer F.Cu) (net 27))
 (segment (start 139.5 54.34) (end 142.5 51.34) (width 0.25) (layer F.Cu) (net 27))
 (segment (start 142.950001 41.849999) (end 143.8 41) (width 0.25) (layer F.Cu) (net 28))
 (segment (start 137.625001 47.174999) (end 142.950001 41.849999) (width 0.25) (layer F.Cu) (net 28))
 (segment (start 137.625001 53.214999) (end 137.625001 47.174999) (width 0.25) (layer F.Cu) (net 28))
 (segment (start 136.5 54.34) (end 137.625001 53.214999) (width 0.25) (layer F.Cu) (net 28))
 (segment (start 158.144999 53.63) (end 158.13 53.615001) (width 0.25) (layer B.Cu) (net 3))
 (segment (start 161 53.63) (end 158.144999 53.63) (width 0.25) (layer B.Cu) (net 3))
 (segment (start 139.849999 77.469999) (end 139 76.62) (width 0.25) (layer F.Cu) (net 4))
 (segment (start 141.45001 79.07001) (end 139.849999 77.469999) (width 0.25) (layer F.Cu) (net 4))
 (segment (start 141.45001 85.195011) (end 141.45001 79.07001) (width 0.25) (layer F.Cu) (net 4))
 (segment (start 142.89 86.635001) (end 141.45001 85.195011) (width 0.25) (layer F.Cu) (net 4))
 (segment (start 139 74.5) (end 139 74.08) (width 0.25) (layer B.Cu) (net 5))
 (segment (start 140.175001 75.675001) (end 139 74.5) (width 0.25) (layer B.Cu) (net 5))
 (segment (start 140.175001 81.380002) (end 140.175001 75.675001) (width 0.25) (layer B.Cu) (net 5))
 (segment (start 142.89 84.095001) (end 140.175001 81.380002) (width 0.25) (layer B.Cu) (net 5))
 (segment (start 139.849999 72.389999) (end 139 71.54) (width 0.25) (layer B.Cu) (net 6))
 (segment (start 140.625011 79.290012) (end 140.625011 73.165011) (width 0.25) (layer B.Cu) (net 6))
 (segment (start 140.625011 73.165011) (end 139.849999 72.389999) (width 0.25) (layer B.Cu) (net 6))
 (segment (start 142.89 81.555001) (end 140.625011 79.290012) (width 0.25) (layer B.Cu) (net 6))
 (segment (start 139 67.665001) (end 142.89 63.775001) (width 0.25) (layer B.Cu) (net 19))
 (segment (start 139 69) (end 139 67.665001) (width 0.25) (layer B.Cu) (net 19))
 (segment (start 156.99863 86.635001) (end 158.13 86.635001) (width 0.25) (layer F.Cu) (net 22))
 (segment (start 152.12292 86.635001) (end 156.99863 86.635001) (width 0.25) (layer F.Cu) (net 22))
 (segment (start 151.78 86.292081) (end 152.12292 86.635001) (width 0.25) (layer F.Cu) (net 22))
 (segment (start 151.78 85.09) (end 151.78 86.292081) (width 0.25) (layer F.Cu) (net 22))
 (segment (start 150.930001 85.939999) (end 151.78 85.09) (width 0.25) (layer F.Cu) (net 22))
 (segment (start 146.775001 86.265001) (end 150.604999 86.265001) (width 0.25) (layer F.Cu) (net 22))
 (segment (start 150.604999 86.265001) (end 150.930001 85.939999) (width 0.25) (layer F.Cu) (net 22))
 (segment (start 146.7 86.19) (end 146.775001 86.265001) (width 0.25) (layer F.Cu) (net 22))
 (segment (start 146.7 85.09) (end 146.7 86.19) (width 0.25) (layer F.Cu) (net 22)))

